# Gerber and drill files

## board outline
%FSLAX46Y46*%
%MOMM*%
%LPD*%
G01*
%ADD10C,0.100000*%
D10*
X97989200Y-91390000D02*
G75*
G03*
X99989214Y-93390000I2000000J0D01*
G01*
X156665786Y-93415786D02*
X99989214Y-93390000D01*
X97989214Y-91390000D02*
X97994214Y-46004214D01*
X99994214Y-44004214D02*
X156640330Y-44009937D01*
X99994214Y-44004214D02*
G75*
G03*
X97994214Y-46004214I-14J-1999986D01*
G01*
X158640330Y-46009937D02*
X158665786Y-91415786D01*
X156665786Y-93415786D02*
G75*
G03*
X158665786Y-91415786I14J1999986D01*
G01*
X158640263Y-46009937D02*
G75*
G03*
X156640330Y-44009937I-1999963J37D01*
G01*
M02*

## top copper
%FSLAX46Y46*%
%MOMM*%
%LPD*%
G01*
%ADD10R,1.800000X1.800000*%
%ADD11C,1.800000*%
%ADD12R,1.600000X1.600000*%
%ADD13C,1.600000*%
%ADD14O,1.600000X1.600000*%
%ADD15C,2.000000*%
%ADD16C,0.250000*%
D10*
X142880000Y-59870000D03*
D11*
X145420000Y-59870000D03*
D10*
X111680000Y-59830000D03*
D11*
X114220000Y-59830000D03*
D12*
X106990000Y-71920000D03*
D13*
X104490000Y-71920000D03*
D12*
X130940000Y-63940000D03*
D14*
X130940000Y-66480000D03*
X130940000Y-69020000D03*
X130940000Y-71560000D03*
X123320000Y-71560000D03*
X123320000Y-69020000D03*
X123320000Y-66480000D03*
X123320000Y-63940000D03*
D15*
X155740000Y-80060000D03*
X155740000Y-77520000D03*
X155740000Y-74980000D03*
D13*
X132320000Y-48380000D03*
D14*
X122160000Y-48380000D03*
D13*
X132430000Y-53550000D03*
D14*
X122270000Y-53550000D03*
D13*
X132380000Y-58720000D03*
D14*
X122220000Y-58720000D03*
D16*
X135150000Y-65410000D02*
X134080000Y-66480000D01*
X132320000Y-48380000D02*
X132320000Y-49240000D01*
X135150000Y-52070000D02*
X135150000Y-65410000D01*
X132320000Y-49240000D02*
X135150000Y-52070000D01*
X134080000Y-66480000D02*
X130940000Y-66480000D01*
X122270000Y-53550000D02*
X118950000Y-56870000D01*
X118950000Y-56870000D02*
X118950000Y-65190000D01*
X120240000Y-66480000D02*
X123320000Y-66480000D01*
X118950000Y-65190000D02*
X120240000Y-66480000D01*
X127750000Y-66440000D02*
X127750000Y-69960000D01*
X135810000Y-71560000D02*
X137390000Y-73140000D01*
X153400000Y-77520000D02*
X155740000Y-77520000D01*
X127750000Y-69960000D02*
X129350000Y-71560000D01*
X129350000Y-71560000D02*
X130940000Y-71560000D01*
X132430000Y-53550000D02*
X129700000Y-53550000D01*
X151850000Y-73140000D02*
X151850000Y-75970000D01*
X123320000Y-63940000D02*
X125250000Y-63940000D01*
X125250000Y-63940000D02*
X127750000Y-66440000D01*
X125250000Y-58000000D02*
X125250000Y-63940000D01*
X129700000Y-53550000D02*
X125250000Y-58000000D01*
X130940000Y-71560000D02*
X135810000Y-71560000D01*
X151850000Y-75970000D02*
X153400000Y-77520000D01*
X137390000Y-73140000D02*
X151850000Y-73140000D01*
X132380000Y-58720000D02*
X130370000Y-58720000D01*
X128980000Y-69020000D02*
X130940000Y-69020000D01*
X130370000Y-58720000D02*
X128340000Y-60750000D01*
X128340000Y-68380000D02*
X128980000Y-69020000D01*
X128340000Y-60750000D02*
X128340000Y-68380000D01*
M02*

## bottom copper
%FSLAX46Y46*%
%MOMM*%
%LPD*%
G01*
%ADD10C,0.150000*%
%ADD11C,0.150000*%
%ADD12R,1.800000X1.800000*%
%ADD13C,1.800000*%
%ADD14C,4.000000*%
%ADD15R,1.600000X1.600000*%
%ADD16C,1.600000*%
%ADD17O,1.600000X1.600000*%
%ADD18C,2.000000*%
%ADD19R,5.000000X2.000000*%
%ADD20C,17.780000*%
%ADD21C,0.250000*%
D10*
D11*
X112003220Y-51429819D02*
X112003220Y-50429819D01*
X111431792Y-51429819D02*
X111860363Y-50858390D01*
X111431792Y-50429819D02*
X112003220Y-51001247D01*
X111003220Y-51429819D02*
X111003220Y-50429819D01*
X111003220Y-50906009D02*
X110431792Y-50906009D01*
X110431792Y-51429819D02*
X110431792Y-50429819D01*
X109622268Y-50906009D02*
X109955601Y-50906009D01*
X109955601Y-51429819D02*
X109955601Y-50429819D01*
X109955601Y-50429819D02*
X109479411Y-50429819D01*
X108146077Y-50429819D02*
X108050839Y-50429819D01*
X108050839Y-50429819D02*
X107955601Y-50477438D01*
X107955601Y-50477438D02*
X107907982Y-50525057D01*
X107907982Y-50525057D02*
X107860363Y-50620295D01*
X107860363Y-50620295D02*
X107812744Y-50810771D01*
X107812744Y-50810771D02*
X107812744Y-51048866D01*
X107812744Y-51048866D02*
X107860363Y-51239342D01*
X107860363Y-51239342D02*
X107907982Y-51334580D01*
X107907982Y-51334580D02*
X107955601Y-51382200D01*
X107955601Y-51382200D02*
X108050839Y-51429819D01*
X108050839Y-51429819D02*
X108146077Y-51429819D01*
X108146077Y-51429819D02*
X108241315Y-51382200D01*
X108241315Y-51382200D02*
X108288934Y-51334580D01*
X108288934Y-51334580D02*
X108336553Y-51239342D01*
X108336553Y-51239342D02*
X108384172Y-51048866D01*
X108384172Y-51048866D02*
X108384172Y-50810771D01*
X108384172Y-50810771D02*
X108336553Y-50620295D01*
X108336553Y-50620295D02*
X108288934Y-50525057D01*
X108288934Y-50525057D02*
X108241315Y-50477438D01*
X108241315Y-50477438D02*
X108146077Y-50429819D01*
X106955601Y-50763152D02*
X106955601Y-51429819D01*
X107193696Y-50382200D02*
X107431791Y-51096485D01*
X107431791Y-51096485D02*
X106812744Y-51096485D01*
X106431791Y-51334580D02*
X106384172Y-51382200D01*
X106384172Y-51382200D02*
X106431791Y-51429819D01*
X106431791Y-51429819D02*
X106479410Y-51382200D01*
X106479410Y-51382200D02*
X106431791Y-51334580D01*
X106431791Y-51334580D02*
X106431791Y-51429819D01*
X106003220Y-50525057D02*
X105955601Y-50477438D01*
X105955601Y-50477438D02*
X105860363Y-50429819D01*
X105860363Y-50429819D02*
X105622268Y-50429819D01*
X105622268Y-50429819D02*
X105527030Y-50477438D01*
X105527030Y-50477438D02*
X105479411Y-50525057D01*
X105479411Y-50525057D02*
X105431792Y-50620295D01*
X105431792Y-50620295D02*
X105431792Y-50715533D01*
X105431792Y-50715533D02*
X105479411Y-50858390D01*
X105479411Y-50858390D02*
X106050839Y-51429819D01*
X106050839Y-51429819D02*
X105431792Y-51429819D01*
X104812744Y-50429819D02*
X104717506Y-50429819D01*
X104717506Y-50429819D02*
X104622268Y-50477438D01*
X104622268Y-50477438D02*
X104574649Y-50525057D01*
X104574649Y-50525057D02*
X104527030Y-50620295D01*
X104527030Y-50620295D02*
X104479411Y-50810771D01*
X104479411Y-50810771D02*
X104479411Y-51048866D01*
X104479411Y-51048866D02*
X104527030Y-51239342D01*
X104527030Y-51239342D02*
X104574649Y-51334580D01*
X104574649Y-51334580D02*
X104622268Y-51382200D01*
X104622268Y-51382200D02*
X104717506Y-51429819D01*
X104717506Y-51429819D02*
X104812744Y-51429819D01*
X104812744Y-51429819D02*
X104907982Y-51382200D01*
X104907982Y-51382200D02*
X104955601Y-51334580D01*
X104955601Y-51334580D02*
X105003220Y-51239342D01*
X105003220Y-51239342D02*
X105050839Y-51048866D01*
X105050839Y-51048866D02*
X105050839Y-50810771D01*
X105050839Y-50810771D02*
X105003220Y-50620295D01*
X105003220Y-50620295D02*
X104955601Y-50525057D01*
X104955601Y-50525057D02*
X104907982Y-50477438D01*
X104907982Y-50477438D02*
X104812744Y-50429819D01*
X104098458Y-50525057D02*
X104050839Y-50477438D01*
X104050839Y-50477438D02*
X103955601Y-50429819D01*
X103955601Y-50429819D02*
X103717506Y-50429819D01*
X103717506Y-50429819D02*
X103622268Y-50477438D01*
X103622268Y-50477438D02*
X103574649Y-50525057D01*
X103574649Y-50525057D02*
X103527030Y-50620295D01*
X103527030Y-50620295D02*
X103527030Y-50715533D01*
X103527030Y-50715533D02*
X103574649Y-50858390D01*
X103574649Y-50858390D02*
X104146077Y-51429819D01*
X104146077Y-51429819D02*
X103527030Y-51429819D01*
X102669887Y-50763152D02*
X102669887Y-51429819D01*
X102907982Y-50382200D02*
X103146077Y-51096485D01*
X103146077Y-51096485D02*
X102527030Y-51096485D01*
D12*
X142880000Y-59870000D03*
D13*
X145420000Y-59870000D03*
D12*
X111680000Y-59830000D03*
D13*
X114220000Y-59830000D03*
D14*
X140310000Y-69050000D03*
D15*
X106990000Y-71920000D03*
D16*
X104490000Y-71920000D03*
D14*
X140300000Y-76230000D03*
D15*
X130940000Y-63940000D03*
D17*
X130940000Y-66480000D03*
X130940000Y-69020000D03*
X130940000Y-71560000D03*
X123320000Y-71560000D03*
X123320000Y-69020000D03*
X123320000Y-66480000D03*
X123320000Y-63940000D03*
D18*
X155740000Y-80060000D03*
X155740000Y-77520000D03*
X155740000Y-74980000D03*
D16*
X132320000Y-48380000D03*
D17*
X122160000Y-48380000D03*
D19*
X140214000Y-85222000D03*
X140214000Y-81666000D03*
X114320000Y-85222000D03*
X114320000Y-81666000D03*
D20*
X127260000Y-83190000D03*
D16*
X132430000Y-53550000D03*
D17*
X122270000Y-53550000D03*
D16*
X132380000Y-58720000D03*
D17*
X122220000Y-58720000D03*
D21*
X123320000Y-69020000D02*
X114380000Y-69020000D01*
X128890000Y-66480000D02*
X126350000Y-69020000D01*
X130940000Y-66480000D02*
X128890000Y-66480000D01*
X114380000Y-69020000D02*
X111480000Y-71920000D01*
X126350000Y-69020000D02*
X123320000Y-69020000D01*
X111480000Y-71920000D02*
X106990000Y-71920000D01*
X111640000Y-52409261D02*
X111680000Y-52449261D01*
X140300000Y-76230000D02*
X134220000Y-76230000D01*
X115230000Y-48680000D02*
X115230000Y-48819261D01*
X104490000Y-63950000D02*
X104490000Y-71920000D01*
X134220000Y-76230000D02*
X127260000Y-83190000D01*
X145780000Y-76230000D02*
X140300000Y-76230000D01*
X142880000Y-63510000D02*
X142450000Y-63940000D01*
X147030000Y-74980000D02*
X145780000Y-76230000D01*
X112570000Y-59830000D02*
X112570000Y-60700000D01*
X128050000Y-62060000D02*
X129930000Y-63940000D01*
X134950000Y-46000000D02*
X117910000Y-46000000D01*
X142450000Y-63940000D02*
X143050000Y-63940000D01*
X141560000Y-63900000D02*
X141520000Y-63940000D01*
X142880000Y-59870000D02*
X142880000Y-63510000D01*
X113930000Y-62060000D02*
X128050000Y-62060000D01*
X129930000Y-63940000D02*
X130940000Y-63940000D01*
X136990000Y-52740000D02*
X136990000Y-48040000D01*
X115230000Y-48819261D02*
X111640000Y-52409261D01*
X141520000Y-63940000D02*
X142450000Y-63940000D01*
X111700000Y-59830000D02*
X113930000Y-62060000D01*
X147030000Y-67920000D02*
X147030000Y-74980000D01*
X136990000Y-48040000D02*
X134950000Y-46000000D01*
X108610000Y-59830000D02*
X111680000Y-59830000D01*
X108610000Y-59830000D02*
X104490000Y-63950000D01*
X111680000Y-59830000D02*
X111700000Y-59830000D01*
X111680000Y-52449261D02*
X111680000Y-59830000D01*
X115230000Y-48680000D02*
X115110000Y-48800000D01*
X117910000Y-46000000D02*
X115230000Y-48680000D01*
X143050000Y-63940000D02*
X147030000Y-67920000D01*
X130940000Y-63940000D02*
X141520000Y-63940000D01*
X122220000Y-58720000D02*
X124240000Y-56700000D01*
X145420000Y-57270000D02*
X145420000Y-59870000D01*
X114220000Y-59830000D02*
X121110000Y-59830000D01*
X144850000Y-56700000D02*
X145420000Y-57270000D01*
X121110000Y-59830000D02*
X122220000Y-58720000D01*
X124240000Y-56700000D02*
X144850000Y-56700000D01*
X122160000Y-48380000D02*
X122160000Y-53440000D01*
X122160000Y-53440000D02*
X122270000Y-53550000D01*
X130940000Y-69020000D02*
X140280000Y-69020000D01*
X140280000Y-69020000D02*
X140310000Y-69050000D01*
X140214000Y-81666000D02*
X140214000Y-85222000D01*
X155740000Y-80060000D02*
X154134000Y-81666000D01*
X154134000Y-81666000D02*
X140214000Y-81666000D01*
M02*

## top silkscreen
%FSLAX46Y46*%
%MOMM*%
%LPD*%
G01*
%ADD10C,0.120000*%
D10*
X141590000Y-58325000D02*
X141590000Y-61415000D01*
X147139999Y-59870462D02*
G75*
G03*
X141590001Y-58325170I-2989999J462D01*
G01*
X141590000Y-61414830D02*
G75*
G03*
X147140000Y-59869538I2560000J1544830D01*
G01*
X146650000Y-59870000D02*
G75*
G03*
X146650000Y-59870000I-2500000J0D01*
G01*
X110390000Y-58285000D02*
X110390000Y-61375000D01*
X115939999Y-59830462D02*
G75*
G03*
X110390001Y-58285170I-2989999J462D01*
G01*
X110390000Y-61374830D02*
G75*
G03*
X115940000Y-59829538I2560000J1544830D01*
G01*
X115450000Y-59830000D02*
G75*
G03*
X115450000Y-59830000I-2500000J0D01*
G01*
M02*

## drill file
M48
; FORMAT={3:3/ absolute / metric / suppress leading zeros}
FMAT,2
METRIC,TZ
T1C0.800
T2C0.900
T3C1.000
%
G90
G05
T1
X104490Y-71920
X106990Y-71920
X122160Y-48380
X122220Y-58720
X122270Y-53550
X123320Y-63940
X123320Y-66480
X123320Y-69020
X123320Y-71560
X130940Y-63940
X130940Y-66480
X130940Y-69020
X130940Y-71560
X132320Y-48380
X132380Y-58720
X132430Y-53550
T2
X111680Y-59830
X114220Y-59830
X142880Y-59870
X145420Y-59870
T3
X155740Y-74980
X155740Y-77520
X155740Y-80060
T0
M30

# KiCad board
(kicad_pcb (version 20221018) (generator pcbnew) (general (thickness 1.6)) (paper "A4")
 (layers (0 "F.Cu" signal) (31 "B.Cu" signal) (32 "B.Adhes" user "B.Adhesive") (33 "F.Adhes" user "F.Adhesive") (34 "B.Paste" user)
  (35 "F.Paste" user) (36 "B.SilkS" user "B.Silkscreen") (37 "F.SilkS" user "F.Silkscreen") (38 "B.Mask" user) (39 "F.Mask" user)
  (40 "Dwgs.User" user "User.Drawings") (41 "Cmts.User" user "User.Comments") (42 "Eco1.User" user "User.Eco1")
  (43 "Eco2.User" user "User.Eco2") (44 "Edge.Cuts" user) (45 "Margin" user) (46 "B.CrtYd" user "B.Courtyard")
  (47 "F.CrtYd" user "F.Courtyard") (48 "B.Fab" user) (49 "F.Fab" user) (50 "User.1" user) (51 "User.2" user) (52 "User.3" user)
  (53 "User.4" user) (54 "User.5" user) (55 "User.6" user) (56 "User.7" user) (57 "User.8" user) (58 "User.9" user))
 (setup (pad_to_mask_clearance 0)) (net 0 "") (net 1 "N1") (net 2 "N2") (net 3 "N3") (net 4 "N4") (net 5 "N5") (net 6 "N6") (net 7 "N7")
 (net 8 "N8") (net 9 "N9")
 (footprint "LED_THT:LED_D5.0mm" (layer "F.Cu") (at 142.88 59.87)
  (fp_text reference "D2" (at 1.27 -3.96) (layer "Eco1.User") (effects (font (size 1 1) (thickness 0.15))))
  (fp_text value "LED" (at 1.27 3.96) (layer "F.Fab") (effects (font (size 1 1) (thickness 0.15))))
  (fp_line (start -1.29 -1.545) (end -1.29 1.545) (stroke (width 0.12) (type solid)) (layer "F.SilkS"))
  (fp_arc (start -1.29 -1.54483) (mid 2.072002 -2.880433) (end 4.26 0.000462) (stroke (width 0.12) (type solid)) (layer "F.SilkS"))
  (fp_arc (start 4.26 -0.000462) (mid 2.072002 2.880433) (end -1.29 1.54483) (stroke (width 0.12) (type solid)) (layer "F.SilkS"))
  (fp_circle (center 1.27 0) (end 3.77 0) (stroke (width 0.12) (type solid)) (fill none) (layer "F.SilkS"))
  (pad "1" thru_hole rect (at 0 0) (size 1.8 1.8) (drill 0.9) (layers "*.Cu" "*.Mask") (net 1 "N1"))
  (pad "2" thru_hole circle (at 2.54 0) (size 1.8 1.8) (drill 0.9) (layers "*.Cu" "*.Mask") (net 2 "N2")))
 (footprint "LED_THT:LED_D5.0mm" (layer "F.Cu") (at 111.68 59.83)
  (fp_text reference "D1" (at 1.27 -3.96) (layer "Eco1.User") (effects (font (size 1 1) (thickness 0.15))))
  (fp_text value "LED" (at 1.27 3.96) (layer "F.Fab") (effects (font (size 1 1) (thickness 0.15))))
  (fp_line (start -1.29 -1.545) (end -1.29 1.545) (stroke (width 0.12) (type solid)) (layer "F.SilkS"))
  (fp_arc (start -1.29 -1.54483) (mid 2.072002 -2.880433) (end 4.26 0.000462) (stroke (width 0.12) (type solid)) (layer "F.SilkS"))
  (fp_arc (start 4.26 -0.000462) (mid 2.072002 2.880433) (end -1.29 1.54483) (stroke (width 0.12) (type solid)) (layer "F.SilkS"))
  (fp_circle (center 1.27 0) (end 3.77 0) (stroke (width 0.12) (type solid)) (fill none) (layer "F.SilkS"))
  (pad "1" thru_hole rect (at 0 0) (size 1.8 1.8) (drill 0.9) (layers "*.Cu" "*.Mask") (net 1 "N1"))
  (pad "2" thru_hole circle (at 2.54 0) (size 1.8 1.8) (drill 0.9) (layers "*.Cu" "*.Mask") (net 2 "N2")))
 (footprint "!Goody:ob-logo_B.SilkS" (layer "F.Cu") (at 151.17 67.66)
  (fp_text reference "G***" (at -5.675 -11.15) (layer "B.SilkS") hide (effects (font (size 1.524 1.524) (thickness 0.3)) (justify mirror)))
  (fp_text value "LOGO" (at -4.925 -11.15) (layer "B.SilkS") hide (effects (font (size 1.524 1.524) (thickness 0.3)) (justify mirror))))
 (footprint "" (layer "F.Cu") (at 140.31 69.05)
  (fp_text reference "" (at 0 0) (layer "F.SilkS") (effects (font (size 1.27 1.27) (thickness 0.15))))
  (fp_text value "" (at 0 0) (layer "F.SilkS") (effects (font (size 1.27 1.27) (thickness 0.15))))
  (pad "1" smd circle (at 0 0 180) (size 4 4) (layers "B.Cu" "B.Paste" "B.Mask") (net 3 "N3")))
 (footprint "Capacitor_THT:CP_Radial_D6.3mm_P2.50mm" (layer "B.Cu") (at 106.99 71.92 180)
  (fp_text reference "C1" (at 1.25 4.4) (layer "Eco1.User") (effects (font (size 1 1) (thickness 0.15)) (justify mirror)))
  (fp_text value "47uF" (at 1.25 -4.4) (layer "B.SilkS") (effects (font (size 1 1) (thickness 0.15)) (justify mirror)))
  (pad "1" thru_hole rect (at 0 0 180) (size 1.6 1.6) (drill 0.8) (layers "*.Cu" "*.Mask") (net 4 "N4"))
  (pad "2" thru_hole circle (at 2.5 0 180) (size 1.6 1.6) (drill 0.8) (layers "*.Cu" "*.Mask") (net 1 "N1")))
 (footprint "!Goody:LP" (layer "B.Cu") (at 140.3 76.23 180)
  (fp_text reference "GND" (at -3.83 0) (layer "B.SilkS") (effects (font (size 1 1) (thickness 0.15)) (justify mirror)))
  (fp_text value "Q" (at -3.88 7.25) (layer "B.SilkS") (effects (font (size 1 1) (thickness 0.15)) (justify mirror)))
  (pad "1" smd circle (at 0 0 180) (size 4 4) (layers "B.Cu" "B.Paste" "B.Mask") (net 1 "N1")))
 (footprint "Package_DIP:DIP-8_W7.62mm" (layer "B.Cu") (at 130.94 63.94 180)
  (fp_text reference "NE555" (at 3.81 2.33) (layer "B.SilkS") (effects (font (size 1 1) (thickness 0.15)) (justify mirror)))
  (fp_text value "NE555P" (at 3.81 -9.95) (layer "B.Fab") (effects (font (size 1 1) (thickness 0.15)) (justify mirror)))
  (pad "1" thru_hole rect (at 0 0 180) (size 1.6 1.6) (drill 0.8) (layers "*.Cu" "*.Mask") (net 1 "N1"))
  (pad "2" thru_hole oval (at 0 -2.54 180) (size 1.6 1.6) (drill 0.8) (layers "*.Cu" "*.Mask") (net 4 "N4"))
  (pad "3" thru_hole oval (at 0 -5.08 180) (size 1.6 1.6) (drill 0.8) (layers "*.Cu" "*.Mask") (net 3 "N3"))
  (pad "4" thru_hole oval (at 0 -7.62 180) (size 1.6 1.6) (drill 0.8) (layers "*.Cu" "*.Mask") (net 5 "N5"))
  (pad "5" thru_hole oval (at 7.62 -7.62 180) (size 1.6 1.6) (drill 0.8) (layers "*.Cu" "*.Mask") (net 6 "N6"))
  (pad "6" thru_hole oval (at 7.62 -5.08 180) (size 1.6 1.6) (drill 0.8) (layers "*.Cu" "*.Mask") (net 4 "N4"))
  (pad "7" thru_hole oval (at 7.62 -2.54 180) (size 1.6 1.6) (drill 0.8) (layers "*.Cu" "*.Mask") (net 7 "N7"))
  (pad "8" thru_hole oval (at 7.62 0 180) (size 1.6 1.6) (drill 0.8) (layers "*.Cu" "*.Mask") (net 5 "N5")))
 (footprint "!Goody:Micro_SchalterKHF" (layer "B.Cu") (at 155.74 80.06 90)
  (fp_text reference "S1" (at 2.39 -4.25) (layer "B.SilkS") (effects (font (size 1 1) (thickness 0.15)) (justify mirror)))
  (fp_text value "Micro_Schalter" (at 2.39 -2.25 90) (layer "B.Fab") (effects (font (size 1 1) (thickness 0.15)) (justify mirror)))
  (pad "1" thru_hole circle (at 0 0 90) (size 2 2) (drill 1) (layers "*.Cu" "*.Mask") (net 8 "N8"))
  (pad "2" thru_hole circle (at 2.54 0 90) (size 2 2) (drill 1) (layers "*.Cu" "*.Mask") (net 5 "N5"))
  (pad "3" thru_hole circle (at 5.08 0 90) (size 2 2) (drill 1) (layers "*.Cu" "*.Mask") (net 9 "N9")))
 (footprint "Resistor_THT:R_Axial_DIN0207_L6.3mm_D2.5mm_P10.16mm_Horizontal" (layer "B.Cu") (at 132.32 48.38 180)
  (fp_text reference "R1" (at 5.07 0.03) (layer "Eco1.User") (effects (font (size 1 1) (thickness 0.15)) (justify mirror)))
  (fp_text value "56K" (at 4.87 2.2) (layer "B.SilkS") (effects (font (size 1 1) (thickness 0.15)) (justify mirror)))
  (pad "1" thru_hole circle (at 0 0 180) (size 1.6 1.6) (drill 0.8) (layers "*.Cu" "*.Mask") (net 4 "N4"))
  (pad "2" thru_hole oval (at 10.16 0 180) (size 1.6 1.6) (drill 0.8) (layers "*.Cu" "*.Mask") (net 7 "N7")))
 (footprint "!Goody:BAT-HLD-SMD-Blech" (layer "B.Cu") (at 127.26 83.19 180)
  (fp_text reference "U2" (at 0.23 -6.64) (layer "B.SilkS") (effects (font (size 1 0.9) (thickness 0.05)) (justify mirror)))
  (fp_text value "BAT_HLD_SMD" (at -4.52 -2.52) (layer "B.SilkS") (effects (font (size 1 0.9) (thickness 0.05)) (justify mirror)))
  (pad "" smd rect (at -12.954 -2.032 180) (size 5 2) (layers "B.Cu" "B.Paste" "B.Mask") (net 8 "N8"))
  (pad "" smd rect (at -12.954 1.524 180) (size 5 2) (layers "B.Cu" "B.Paste" "B.Mask") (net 8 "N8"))
  (pad "1" smd rect (at 12.94 -2.032 180) (size 5 2) (layers "B.Cu" "B.Paste" "B.Mask"))
  (pad "1" smd rect (at 12.94 1.524 180) (size 5 2) (layers "B.Cu" "B.Paste" "B.Mask"))
  (pad "2" smd circle (at 0 0 180) (size 17.78 17.78) (layers "B.Cu" "B.Paste" "B.Mask") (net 1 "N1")))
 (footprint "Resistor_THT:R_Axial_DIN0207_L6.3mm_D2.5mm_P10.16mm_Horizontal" (layer "B.Cu") (at 132.43 53.55 180)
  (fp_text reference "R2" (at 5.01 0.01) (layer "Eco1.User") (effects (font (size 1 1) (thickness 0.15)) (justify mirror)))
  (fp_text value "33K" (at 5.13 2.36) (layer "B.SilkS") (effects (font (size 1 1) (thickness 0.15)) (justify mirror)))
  (pad "1" thru_hole circle (at 0 0 180) (size 1.6 1.6) (drill 0.8) (layers "*.Cu" "*.Mask") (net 5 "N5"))
  (pad "2" thru_hole oval (at 10.16 0 180) (size 1.6 1.6) (drill 0.8) (layers "*.Cu" "*.Mask") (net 7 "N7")))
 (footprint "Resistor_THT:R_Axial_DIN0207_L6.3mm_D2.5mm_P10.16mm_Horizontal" (layer "B.Cu") (at 132.38 58.72 180)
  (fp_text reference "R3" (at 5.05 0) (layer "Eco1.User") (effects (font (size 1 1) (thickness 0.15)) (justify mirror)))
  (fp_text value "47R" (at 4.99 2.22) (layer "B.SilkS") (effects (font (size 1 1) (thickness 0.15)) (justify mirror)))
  (pad "1" thru_hole circle (at 0 0 180) (size 1.6 1.6) (drill 0.8) (layers "*.Cu" "*.Mask") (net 3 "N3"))
  (pad "2" thru_hole oval (at 10.16 0 180) (size 1.6 1.6) (drill 0.8) (layers "*.Cu" "*.Mask") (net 2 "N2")))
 (gr_arc (start 99.989214 93.39) (mid 98.575 92.804214) (end 97.989214 91.39) (stroke (width 0.1) (type default)) (layer "Edge.Cuts"))
 (gr_line (start 156.665786 93.415786) (end 99.989214 93.39) (stroke (width 0.1) (type default)) (layer "Edge.Cuts"))
 (gr_line (start 97.989214 91.39) (end 97.994214 46.004214) (stroke (width 0.1) (type default)) (layer "Edge.Cuts"))
 (gr_line (start 99.994214 44.004214) (end 156.64033 44.009937) (stroke (width 0.1) (type default)) (layer "Edge.Cuts"))
 (gr_arc (start 97.994214 46.004214) (mid 98.58 44.59) (end 99.994214 44.004214) (stroke (width 0.1) (type default)) (layer "Edge.Cuts"))
 (gr_line (start 158.64033 46.009937) (end 158.665786 91.415786) (stroke (width 0.1) (type default)) (layer "Edge.Cuts"))
 (gr_arc (start 158.665786 91.415786) (mid 158.08 92.83) (end 156.665786 93.415786) (stroke (width 0.1) (type default)) (layer "Edge.Cuts"))
 (gr_arc (start 156.64033 44.009937) (mid 158.054544 44.595723) (end 158.64033 46.009937) (stroke (width 0.1) (type default))
  (layer "Edge.Cuts"))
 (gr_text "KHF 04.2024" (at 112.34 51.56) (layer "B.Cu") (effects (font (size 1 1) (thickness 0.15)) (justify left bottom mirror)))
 (segment (start 135.15 65.41) (end 134.08 66.48) (width 0.25) (layer "F.Cu") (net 4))
 (segment (start 132.32 48.38) (end 132.32 49.24) (width 0.25) (layer "F.Cu") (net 4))
 (segment (start 135.15 52.07) (end 135.15 65.41) (width 0.25) (layer "F.Cu") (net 4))
 (segment (start 132.32 49.24) (end 135.15 52.07) (width 0.25) (layer "F.Cu") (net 4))
 (segment (start 134.08 66.48) (end 130.94 66.48) (width 0.25) (layer "F.Cu") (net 4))
 (segment (start 123.32 69.02) (end 114.38 69.02) (width 0.25) (layer "B.Cu") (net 4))
 (segment (start 128.89 66.48) (end 126.35 69.02) (width 0.25) (layer "B.Cu") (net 4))
 (segment (start 130.94 66.48) (end 128.89 66.48) (width 0.25) (layer "B.Cu") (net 4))
 (segment (start 114.38 69.02) (end 111.48 71.92) (width 0.25) (layer "B.Cu") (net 4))
 (segment (start 126.35 69.02) (end 123.32 69.02) (width 0.25) (layer "B.Cu") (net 4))
 (segment (start 111.48 71.92) (end 106.99 71.92) (width 0.25) (layer "B.Cu") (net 4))
 (segment (start 111.64 52.409261) (end 111.68 52.449261) (width 0.25) (layer "B.Cu") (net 1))
 (segment (start 140.3 76.23) (end 134.22 76.23) (width 0.25) (layer "B.Cu") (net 1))
 (segment (start 115.23 48.68) (end 115.23 48.819261) (width 0.25) (layer "B.Cu") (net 1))
 (segment (start 104.49 63.95) (end 104.49 71.92) (width 0.25) (layer "B.Cu") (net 1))
 (segment (start 134.22 76.23) (end 127.26 83.19) (width 0.25) (layer "B.Cu") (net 1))
 (segment (start 145.78 76.23) (end 140.3 76.23) (width 0.25) (layer "B.Cu") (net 1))
 (segment (start 142.88 63.51) (end 142.45 63.94) (width 0.25) (layer "B.Cu") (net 1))
 (segment (start 147.03 74.98) (end 145.78 76.23) (width 0.25) (layer "B.Cu") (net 1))
 (segment (start 112.57 59.83) (end 112.57 60.7) (width 0.25) (layer "B.Cu") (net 1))
 (segment (start 128.05 62.06) (end 129.93 63.94) (width 0.25) (layer "B.Cu") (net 1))
 (segment (start 134.95 46) (end 117.91 46) (width 0.25) (layer "B.Cu") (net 1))
 (segment (start 142.45 63.94) (end 143.05 63.94) (width 0.25) (layer "B.Cu") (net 1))
 (segment (start 141.56 63.9) (end 141.52 63.94) (width 0.25) (layer "B.Cu") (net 1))
 (segment (start 142.88 59.87) (end 142.88 63.51) (width 0.25) (layer "B.Cu") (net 1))
 (segment (start 113.93 62.06) (end 128.05 62.06) (width 0.25) (layer "B.Cu") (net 1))
 (segment (start 129.93 63.94) (end 130.94 63.94) (width 0.25) (layer "B.Cu") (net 1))
 (segment (start 136.99 52.74) (end 136.99 48.04) (width 0.25) (layer "B.Cu") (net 1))
 (segment (start 115.23 48.819261) (end 111.64 52.409261) (width 0.25) (layer "B.Cu") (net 1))
 (segment (start 141.52 63.94) (end 142.45 63.94) (width 0.25) (layer "B.Cu") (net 1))
 (segment (start 111.7 59.83) (end 113.93 62.06) (width 0.25) (layer "B.Cu") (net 1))
 (segment (start 147.03 67.92) (end 147.03 74.98) (width 0.25) (layer "B.Cu") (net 1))
 (segment (start 136.99 48.04) (end 134.95 46) (width 0.25) (layer "B.Cu") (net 1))
 (segment (start 108.61 59.83) (end 111.68 59.83) (width 0.25) (layer "B.Cu") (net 1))
 (segment (start 108.61 59.83) (end 104.49 63.95) (width 0.25) (layer "B.Cu") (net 1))
 (segment (start 111.68 59.83) (end 111.7 59.83) (width 0.25) (layer "B.Cu") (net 1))
 (segment (start 111.68 52.449261) (end 111.68 59.83) (width 0.25) (layer "B.Cu") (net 1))
 (segment (start 115.23 48.68) (end 115.11 48.8) (width 0.25) (layer "B.Cu") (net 1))
 (segment (start 117.91 46) (end 115.23 48.68) (width 0.25) (layer "B.Cu") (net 1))
 (segment (start 143.05 63.94) (end 147.03 67.92) (width 0.25) (layer "B.Cu") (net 1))
 (segment (start 130.94 63.94) (end 141.52 63.94) (width 0.25) (layer "B.Cu") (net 1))
 (segment (start 122.22 58.72) (end 124.24 56.7) (width 0.25) (layer "B.Cu") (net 2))
 (segment (start 145.42 57.27) (end 145.42 59.87) (width 0.25) (layer "B.Cu") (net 2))
 (segment (start 114.22 59.83) (end 121.11 59.83) (width 0.25) (layer "B.Cu") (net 2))
 (segment (start 144.85 56.7) (end 145.42 57.27) (width 0.25) (layer "B.Cu") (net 2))
 (segment (start 121.11 59.83) (end 122.22 58.72) (width 0.25) (layer "B.Cu") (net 2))
 (segment (start 124.24 56.7) (end 144.85 56.7) (width 0.25) (layer "B.Cu") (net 2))
 (segment (start 122.27 53.55) (end 118.95 56.87) (width 0.25) (layer "F.Cu") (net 7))
 (segment (start 118.95 56.87) (end 118.95 65.19) (width 0.25) (layer "F.Cu") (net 7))
 (segment (start 120.24 66.48) (end 123.32 66.48) (width 0.25) (layer "F.Cu") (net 7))
 (segment (start 118.95 65.19) (end 120.24 66.48) (width 0.25) (layer "F.Cu") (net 7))
 (segment (start 122.16 48.38) (end 122.16 53.44) (width 0.25) (layer "B.Cu") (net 7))
 (segment (start 122.16 53.44) (end 122.27 53.55) (width 0.25) (layer "B.Cu") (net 7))
 (segment (start 127.75 66.44) (end 127.75 69.96) (width 0.25) (layer "F.Cu") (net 5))
 (segment (start 135.81 71.56) (end 137.39 73.14) (width 0.25) (layer "F.Cu") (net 5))
 (segment (start 153.4 77.52) (end 155.74 77.52) (width 0.25) (layer "F.Cu") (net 5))
 (segment (start 127.75 69.96) (end 129.35 71.56) (width 0.25) (layer "F.Cu") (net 5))
 (segment (start 129.35 71.56) (end 130.94 71.56) (width 0.25) (layer "F.Cu") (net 5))
 (segment (start 132.43 53.55) (end 129.7 53.55) (width 0.25) (layer "F.Cu") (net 5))
 (segment (start 151.85 73.14) (end 151.85 75.97) (width 0.25) (layer "F.Cu") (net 5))
 (segment (start 123.32 63.94) (end 125.25 63.94) (width 0.25) (layer "F.Cu") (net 5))
 (segment (start 125.25 63.94) (end 127.75 66.44) (width 0.25) (layer "F.Cu") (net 5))
 (segment (start 125.25 58) (end 125.25 63.94) (width 0.25) (layer "F.Cu") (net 5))
 (segment (start 129.7 53.55) (end 125.25 58) (width 0.25) (layer "F.Cu") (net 5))
 (segment (start 130.94 71.56) (end 135.81 71.56) (width 0.25) (layer "F.Cu") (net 5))
 (segment (start 151.85 75.97) (end 153.4 77.52) (width 0.25) (layer "F.Cu") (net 5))
 (segment (start 137.39 73.14) (end 151.85 73.14) (width 0.25) (layer "F.Cu") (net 5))
 (segment (start 132.38 58.72) (end 130.37 58.72) (width 0.25) (layer "F.Cu") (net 3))
 (segment (start 128.98 69.02) (end 130.94 69.02) (width 0.25) (layer "F.Cu") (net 3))
 (segment (start 130.37 58.72) (end 128.34 60.75) (width 0.25) (layer "F.Cu") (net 3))
 (segment (start 128.34 68.38) (end 128.98 69.02) (width 0.25) (layer "F.Cu") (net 3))
 (segment (start 128.34 60.75) (end 128.34 68.38) (width 0.25) (layer "F.Cu") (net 3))
 (segment (start 130.94 69.02) (end 140.28 69.02) (width 0.25) (layer "B.Cu") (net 3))
 (segment (start 140.28 69.02) (end 140.31 69.05) (width 0.25) (layer "B.Cu") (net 3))
 (segment (start 140.214 81.666) (end 140.214 85.222) (width 0.25) (layer "B.Cu") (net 8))
 (segment (start 155.74 80.06) (end 154.134 81.666) (width 0.25) (layer "B.Cu") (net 8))
 (segment (start 154.134 81.666) (end 140.214 81.666) (width 0.25) (layer "B.Cu") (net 8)))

